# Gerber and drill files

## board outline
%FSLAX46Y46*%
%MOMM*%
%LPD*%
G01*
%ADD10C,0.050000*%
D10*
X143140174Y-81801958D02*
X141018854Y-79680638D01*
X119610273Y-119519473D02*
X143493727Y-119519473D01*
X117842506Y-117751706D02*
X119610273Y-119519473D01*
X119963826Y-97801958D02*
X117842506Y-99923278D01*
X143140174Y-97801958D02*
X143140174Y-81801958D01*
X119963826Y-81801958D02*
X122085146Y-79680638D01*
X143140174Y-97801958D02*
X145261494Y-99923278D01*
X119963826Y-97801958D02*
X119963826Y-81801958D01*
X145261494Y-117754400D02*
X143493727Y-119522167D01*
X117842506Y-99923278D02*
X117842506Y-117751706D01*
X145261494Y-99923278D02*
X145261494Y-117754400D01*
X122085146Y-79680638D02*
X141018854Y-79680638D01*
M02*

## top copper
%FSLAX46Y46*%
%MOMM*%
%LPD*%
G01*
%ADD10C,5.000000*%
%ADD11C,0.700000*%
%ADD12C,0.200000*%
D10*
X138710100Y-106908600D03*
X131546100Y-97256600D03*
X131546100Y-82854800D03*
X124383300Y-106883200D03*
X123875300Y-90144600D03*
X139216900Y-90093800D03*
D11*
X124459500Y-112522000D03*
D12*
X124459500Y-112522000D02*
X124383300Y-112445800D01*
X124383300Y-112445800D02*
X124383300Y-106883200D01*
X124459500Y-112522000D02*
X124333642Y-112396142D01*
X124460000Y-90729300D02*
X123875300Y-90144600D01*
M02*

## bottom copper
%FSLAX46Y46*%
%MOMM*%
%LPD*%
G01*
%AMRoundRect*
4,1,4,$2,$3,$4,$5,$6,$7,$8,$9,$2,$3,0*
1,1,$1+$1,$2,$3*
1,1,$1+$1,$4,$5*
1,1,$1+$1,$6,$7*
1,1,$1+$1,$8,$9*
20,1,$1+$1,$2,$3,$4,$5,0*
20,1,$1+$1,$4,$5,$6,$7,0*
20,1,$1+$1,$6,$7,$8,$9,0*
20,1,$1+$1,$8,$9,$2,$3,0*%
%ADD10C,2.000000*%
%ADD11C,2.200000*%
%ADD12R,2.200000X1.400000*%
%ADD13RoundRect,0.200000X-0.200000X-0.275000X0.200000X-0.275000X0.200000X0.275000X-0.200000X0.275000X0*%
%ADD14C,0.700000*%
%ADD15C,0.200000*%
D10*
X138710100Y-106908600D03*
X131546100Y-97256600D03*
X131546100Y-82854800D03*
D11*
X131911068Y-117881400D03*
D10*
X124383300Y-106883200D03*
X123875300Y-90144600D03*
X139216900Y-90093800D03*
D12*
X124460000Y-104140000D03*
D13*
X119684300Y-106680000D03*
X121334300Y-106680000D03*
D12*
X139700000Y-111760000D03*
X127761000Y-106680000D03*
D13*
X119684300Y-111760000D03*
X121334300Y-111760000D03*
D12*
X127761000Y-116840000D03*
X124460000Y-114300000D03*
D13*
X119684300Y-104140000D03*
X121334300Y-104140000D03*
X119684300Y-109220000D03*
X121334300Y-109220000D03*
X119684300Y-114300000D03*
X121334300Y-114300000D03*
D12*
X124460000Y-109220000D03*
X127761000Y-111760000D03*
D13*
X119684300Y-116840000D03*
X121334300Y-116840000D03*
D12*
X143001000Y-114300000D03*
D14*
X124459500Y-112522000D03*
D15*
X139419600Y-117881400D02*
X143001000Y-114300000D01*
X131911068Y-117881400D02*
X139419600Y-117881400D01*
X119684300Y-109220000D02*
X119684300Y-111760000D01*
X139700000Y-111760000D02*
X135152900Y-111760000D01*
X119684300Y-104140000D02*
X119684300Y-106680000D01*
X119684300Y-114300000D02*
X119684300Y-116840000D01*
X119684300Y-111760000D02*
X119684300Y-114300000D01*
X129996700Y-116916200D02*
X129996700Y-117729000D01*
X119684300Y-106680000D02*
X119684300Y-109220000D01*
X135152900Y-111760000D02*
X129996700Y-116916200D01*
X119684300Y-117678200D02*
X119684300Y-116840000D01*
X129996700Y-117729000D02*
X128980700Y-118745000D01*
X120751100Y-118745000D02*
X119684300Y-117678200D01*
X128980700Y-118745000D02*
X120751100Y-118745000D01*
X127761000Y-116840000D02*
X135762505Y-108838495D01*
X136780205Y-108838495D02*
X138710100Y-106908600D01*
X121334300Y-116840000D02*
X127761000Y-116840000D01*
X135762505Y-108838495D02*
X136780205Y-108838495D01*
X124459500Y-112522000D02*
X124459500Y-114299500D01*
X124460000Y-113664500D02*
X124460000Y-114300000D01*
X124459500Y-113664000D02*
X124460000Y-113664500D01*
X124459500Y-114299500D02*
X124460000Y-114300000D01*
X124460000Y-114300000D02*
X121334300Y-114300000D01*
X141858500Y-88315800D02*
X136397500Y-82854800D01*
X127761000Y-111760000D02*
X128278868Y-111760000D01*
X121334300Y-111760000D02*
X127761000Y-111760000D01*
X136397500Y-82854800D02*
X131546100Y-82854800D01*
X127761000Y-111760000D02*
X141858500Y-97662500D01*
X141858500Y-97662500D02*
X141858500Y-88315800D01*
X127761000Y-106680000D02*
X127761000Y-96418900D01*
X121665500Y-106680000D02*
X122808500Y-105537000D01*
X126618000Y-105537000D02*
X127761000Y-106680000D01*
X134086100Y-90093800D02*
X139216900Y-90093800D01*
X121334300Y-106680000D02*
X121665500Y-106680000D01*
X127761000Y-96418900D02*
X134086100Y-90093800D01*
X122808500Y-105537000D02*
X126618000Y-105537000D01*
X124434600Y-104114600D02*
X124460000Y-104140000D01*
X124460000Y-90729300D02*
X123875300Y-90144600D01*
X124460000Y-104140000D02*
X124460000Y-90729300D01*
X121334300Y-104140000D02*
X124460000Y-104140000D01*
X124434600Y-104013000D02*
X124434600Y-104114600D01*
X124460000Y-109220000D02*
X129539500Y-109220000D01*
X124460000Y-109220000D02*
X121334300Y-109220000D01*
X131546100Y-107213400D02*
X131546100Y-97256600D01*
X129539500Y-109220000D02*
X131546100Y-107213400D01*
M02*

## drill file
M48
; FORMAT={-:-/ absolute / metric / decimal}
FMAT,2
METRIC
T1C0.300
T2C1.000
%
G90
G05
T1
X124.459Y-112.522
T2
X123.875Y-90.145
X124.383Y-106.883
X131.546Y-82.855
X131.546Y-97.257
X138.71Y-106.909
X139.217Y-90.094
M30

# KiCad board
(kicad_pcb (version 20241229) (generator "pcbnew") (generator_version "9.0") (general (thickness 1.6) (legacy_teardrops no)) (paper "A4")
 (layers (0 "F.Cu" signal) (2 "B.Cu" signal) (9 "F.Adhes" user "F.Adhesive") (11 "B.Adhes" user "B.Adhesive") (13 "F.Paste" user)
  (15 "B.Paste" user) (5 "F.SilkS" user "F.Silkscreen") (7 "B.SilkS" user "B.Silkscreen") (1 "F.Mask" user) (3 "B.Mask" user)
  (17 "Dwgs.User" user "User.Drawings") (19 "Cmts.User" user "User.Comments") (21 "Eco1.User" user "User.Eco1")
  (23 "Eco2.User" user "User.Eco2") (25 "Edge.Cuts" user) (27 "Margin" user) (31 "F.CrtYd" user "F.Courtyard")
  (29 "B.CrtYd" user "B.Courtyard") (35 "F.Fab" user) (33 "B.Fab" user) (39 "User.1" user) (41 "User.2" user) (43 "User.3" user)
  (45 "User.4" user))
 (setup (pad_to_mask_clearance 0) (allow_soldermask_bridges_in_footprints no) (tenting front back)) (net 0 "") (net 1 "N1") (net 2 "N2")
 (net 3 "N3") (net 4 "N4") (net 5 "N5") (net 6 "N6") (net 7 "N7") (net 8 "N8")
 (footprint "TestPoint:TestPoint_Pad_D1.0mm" (layer "F.Cu") (at 138.7101 106.9086 90)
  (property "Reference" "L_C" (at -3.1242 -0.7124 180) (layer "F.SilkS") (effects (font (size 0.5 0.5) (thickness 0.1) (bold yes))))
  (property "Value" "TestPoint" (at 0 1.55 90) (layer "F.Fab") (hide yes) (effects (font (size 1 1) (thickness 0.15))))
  (pad "1" thru_hole circle (at 0 0 90) (size 5 5) (drill 1) (layers "*.Cu" "*.Mask") (remove_unused_layers no) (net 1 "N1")
   (padstack (mode front_inner_back) (layer "Inner" (shape circle) (size 5 5) (zone_connect -1))
    (layer "B.Cu" (shape circle) (size 2 2) (zone_connect -1)))))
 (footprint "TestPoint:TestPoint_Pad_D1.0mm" (layer "F.Cu") (at 131.5461 97.2566 90)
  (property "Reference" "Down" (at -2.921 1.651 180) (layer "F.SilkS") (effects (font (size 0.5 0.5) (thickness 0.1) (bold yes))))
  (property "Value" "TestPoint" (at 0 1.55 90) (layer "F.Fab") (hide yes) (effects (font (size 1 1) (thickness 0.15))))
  (pad "1" thru_hole circle (at 0 0 180) (size 5 5) (drill 1) (layers "*.Cu" "*.Mask") (remove_unused_layers no) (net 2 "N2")
   (padstack (mode front_inner_back) (layer "Inner" (shape circle) (size 5 5) (zone_connect -1))
    (layer "B.Cu" (shape circle) (size 2 2) (zone_connect -1)))))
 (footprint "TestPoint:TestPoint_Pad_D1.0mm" (layer "F.Cu") (at 131.5461 82.8548 90)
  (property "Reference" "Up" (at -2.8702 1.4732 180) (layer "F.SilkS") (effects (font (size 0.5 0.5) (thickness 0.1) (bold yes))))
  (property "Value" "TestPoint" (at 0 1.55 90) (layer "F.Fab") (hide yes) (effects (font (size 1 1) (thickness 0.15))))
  (pad "1" thru_hole circle (at 0 0) (size 5 5) (drill 1) (layers "*.Cu" "*.Mask") (remove_unused_layers no) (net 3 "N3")
   (padstack (mode front_inner_back) (layer "Inner" (shape circle) (size 5 5) (zone_connect -1))
    (layer "B.Cu" (shape circle) (size 2 2) (zone_connect -1)))))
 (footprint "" (layer "F.Cu") (at 131.911068 117.8814)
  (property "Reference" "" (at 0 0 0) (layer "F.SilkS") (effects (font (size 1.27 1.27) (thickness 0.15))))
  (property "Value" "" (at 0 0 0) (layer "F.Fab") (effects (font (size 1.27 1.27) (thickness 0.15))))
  (pad "1" smd circle (at 0 0 180) (size 2.2 2.2) (layers "B.Cu" "B.Mask") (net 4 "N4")))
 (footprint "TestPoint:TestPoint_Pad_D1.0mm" (layer "F.Cu") (at 124.3833 106.8832 90)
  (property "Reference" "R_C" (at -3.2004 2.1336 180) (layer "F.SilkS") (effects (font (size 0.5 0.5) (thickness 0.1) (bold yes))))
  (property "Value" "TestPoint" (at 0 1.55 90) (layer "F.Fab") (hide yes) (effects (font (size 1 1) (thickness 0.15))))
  (pad "1" thru_hole circle (at 0 0 90) (size 5 5) (drill 1) (layers "*.Cu" "*.Mask") (remove_unused_layers no) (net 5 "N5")
   (padstack (mode front_inner_back) (layer "Inner" (shape circle) (size 5 5) (zone_connect -1))
    (layer "B.Cu" (shape circle) (size 2 2) (zone_connect -1)))))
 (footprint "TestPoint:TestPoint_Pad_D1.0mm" (layer "F.Cu") (at 123.8753 90.1446 90)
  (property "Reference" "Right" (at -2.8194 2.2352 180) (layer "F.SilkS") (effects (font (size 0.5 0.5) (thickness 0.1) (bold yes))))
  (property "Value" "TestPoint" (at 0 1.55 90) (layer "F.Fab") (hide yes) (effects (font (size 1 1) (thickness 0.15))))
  (pad "1" thru_hole circle (at 0 0 270) (size 5 5) (drill 1) (layers "*.Cu" "*.Mask") (remove_unused_layers no) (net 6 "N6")
   (teardrops (best_length_ratio 0.5) (max_length 1) (best_width_ratio 0.7) (max_width 2) (curved_edges no) (filter_ratio 0.9) (enabled no)
    (allow_two_segments yes) (prefer_zone_connections yes))
   (padstack (mode front_inner_back) (layer "Inner" (shape circle) (size 5 5) (zone_connect -1))
    (layer "B.Cu" (shape circle) (size 2 2) (zone_connect -1)))))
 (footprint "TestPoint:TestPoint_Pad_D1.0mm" (layer "F.Cu") (at 139.2169 90.0938 90)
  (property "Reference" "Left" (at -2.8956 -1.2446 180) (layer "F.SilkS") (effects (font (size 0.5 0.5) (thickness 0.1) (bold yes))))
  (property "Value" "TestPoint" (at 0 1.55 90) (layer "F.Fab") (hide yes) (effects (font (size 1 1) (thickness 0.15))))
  (pad "1" thru_hole circle (at 0 0 90) (size 5 5) (drill 1) (layers "*.Cu" "*.Mask") (remove_unused_layers no) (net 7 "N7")
   (padstack (mode front_inner_back) (layer "Inner" (shape circle) (size 5 5) (zone_connect -1))
    (layer "B.Cu" (shape circle) (size 2 2) (zone_connect -1)))))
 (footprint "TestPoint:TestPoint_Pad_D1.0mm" (layer "B.Cu") (at 124.46 104.14 180)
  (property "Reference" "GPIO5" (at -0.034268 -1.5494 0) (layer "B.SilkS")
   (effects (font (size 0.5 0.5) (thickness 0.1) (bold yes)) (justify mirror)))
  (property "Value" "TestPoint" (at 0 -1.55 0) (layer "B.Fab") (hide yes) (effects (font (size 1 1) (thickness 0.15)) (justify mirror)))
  (pad "1" smd rect (at 0 0 180) (size 2.2 1.4) (layers "B.Cu" "B.Mask") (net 6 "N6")))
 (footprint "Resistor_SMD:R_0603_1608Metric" (layer "B.Cu") (at 120.5093 106.68)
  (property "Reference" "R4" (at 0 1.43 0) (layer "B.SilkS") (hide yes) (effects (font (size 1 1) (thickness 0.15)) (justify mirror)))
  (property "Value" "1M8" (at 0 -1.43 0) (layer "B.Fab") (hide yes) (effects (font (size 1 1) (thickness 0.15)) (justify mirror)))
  (pad "1" smd roundrect (at -0.825 0) (size 0.8 0.95) (layers "B.Cu" "B.Mask" "B.Paste") (roundrect_rratio 0.25) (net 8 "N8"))
  (pad "2" smd roundrect (at 0.825 0) (size 0.8 0.95) (layers "B.Cu" "B.Mask" "B.Paste") (roundrect_rratio 0.25) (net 7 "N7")))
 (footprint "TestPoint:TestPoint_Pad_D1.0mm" (layer "B.Cu") (at 139.7 111.76)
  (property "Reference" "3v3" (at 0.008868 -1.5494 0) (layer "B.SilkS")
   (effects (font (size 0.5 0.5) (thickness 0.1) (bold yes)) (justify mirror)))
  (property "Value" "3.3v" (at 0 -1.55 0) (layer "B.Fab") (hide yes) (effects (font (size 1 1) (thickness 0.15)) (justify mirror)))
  (pad "1" smd rect (at 0 0) (size 2.2 1.4) (layers "B.Cu" "B.Mask") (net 8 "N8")))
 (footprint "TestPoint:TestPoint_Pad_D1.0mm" (layer "B.Cu") (at 127.761 106.68 180)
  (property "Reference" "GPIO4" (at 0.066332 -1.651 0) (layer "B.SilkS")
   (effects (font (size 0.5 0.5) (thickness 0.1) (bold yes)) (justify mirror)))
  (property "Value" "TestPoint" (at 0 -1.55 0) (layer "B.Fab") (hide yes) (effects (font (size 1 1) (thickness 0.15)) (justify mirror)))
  (pad "1" smd rect (at 0 0 180) (size 2.2 1.4) (layers "B.Cu" "B.Mask") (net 7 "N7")))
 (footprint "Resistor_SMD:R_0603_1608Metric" (layer "B.Cu") (at 120.5093 111.76)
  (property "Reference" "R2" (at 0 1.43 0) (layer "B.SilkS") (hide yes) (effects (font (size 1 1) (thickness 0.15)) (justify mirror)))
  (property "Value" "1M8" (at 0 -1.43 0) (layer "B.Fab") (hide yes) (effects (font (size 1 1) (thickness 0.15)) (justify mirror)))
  (pad "1" smd roundrect (at -0.825 0) (size 0.8 0.95) (layers "B.Cu" "B.Mask" "B.Paste") (roundrect_rratio 0.25) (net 8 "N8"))
  (pad "2" smd roundrect (at 0.825 0) (size 0.8 0.95) (layers "B.Cu" "B.Mask" "B.Paste") (roundrect_rratio 0.25) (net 3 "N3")))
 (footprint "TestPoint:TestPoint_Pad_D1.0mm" (layer "B.Cu") (at 127.761 116.84 180)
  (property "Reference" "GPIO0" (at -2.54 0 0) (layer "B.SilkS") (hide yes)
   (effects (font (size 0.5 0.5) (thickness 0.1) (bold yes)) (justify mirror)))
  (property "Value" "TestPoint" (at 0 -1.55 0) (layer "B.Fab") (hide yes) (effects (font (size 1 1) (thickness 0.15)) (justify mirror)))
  (pad "1" smd rect (at 0 0 180) (size 2.2 1.4) (layers "B.Cu" "B.Mask") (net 1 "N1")))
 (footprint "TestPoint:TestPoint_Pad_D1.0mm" (layer "B.Cu") (at 124.46 114.3 180)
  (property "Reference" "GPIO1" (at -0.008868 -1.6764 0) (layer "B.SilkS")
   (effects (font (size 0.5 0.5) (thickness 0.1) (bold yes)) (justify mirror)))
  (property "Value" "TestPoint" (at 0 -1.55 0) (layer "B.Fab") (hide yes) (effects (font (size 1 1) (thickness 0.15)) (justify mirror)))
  (pad "1" smd rect (at 0 0 180) (size 2.2 1.4) (layers "B.Cu" "B.Mask") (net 5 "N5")))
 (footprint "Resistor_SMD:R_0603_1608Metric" (layer "B.Cu") (at 120.5093 104.14)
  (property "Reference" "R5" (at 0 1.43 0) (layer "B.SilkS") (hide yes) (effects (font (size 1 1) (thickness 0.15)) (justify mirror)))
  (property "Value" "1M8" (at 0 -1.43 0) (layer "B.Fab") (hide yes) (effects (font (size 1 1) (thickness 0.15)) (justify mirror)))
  (pad "1" smd roundrect (at -0.825 0) (size 0.8 0.95) (layers "B.Cu" "B.Mask" "B.Paste") (roundrect_rratio 0.25) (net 8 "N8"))
  (pad "2" smd roundrect (at 0.825 0) (size 0.8 0.95) (layers "B.Cu" "B.Mask" "B.Paste") (roundrect_rratio 0.25) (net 6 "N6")))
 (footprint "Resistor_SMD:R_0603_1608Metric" (layer "B.Cu") (at 120.5093 109.22)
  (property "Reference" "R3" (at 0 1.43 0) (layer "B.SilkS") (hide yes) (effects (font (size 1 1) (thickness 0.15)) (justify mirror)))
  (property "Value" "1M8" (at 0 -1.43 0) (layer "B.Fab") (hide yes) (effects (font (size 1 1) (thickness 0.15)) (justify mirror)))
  (pad "1" smd roundrect (at -0.825 0) (size 0.8 0.95) (layers "B.Cu" "B.Mask" "B.Paste") (roundrect_rratio 0.25) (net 8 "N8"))
  (pad "2" smd roundrect (at 0.825 0) (size 0.8 0.95) (layers "B.Cu" "B.Mask" "B.Paste") (roundrect_rratio 0.25) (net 2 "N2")))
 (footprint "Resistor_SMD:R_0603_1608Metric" (layer "B.Cu") (at 120.5093 114.3)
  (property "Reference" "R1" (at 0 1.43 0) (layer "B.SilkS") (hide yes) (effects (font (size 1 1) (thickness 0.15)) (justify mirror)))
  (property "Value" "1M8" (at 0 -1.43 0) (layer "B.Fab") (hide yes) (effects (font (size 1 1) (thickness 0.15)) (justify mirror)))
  (pad "1" smd roundrect (at -0.825 0) (size 0.8 0.95) (layers "B.Cu" "B.Mask" "B.Paste") (roundrect_rratio 0.25) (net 8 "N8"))
  (pad "2" smd roundrect (at 0.825 0) (size 0.8 0.95) (layers "B.Cu" "B.Mask" "B.Paste") (roundrect_rratio 0.25) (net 5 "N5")))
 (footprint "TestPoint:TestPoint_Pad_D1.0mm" (layer "B.Cu") (at 124.46 109.22 180)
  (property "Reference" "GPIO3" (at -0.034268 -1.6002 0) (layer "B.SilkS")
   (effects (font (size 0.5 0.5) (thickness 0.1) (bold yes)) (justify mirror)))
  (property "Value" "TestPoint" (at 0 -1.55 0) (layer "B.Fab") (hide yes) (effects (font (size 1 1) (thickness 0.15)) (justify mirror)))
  (pad "1" smd rect (at 0 0 180) (size 2.2 1.4) (layers "B.Cu" "B.Mask") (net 2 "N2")))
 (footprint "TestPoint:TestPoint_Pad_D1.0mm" (layer "B.Cu") (at 127.761 111.76 180)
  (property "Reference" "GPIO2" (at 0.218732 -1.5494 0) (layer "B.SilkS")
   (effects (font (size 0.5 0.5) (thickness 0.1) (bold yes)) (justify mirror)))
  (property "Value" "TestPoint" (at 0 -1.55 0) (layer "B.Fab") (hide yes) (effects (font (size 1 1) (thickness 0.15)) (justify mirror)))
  (pad "1" smd rect (at 0 0 180) (size 2.2 1.4) (layers "B.Cu" "B.Mask") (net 3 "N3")))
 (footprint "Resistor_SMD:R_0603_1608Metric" (layer "B.Cu") (at 120.5093 116.84)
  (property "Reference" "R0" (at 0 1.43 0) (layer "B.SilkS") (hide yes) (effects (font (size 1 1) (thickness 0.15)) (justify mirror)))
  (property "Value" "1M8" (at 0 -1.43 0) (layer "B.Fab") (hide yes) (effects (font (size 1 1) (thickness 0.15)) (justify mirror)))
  (pad "1" smd roundrect (at -0.825 0) (size 0.8 0.95) (layers "B.Cu" "B.Mask" "B.Paste") (roundrect_rratio 0.25) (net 8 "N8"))
  (pad "2" smd roundrect (at 0.825 0) (size 0.8 0.95) (layers "B.Cu" "B.Mask" "B.Paste") (roundrect_rratio 0.25) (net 1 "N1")))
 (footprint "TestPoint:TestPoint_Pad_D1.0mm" (layer "B.Cu") (at 143.001 114.3)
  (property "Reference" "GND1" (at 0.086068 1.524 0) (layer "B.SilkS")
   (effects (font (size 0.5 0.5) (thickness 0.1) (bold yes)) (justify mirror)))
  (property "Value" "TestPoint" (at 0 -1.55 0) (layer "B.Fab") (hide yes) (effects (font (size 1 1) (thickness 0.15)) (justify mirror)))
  (pad "1" smd rect (at 0 0) (size 2.2 1.4) (layers "B.Cu" "B.Mask") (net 4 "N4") (clearance 0.1)))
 (gr_line (start 143.140174 81.801958) (end 141.018854 79.680638) (stroke (width 0.05) (type solid)) (layer "Edge.Cuts"))
 (gr_line (start 119.610273 119.519473) (end 143.493727 119.519473) (stroke (width 0.05) (type default)) (layer "Edge.Cuts"))
 (gr_line (start 117.842506 117.751706) (end 119.610273 119.519473) (stroke (width 0.05) (type solid)) (layer "Edge.Cuts"))
 (gr_line (start 119.963826 97.801958) (end 117.842506 99.923278) (stroke (width 0.05) (type solid)) (layer "Edge.Cuts"))
 (gr_line (start 143.140174 97.801958) (end 143.140174 81.801958) (stroke (width 0.05) (type solid)) (layer "Edge.Cuts"))
 (gr_line (start 119.963826 81.801958) (end 122.085146 79.680638) (stroke (width 0.05) (type solid)) (layer "Edge.Cuts"))
 (gr_line (start 143.140174 97.801958) (end 145.261494 99.923278) (stroke (width 0.05) (type solid)) (layer "Edge.Cuts"))
 (gr_line (start 119.963826 97.801958) (end 119.963826 81.801958) (stroke (width 0.05) (type solid)) (layer "Edge.Cuts"))
 (gr_line (start 145.261494 117.7544) (end 143.493727 119.522167) (stroke (width 0.05) (type solid)) (layer "Edge.Cuts"))
 (gr_line (start 117.842506 99.923278) (end 117.842506 117.751706) (stroke (width 0.05) (type default)) (layer "Edge.Cuts"))
 (gr_line (start 145.261494 99.923278) (end 145.261494 117.7544) (stroke (width 0.05) (type default)) (layer "Edge.Cuts"))
 (gr_line (start 122.085146 79.680638) (end 141.018854 79.680638) (stroke (width 0.05) (type default)) (layer "Edge.Cuts"))
 (segment (start 139.4196 117.8814) (end 143.001 114.3) (width 0.2) (layer "B.Cu") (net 4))
 (segment (start 131.911068 117.8814) (end 139.4196 117.8814) (width 0.2) (layer "B.Cu") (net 4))
 (segment (start 119.6843 109.22) (end 119.6843 111.76) (width 0.2) (layer "B.Cu") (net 8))
 (segment (start 139.7 111.76) (end 135.1529 111.76) (width 0.2) (layer "B.Cu") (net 8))
 (segment (start 119.6843 104.14) (end 119.6843 106.68) (width 0.2) (layer "B.Cu") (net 8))
 (segment (start 119.6843 114.3) (end 119.6843 116.84) (width 0.2) (layer "B.Cu") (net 8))
 (segment (start 119.6843 111.76) (end 119.6843 114.3) (width 0.2) (layer "B.Cu") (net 8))
 (segment (start 129.9967 116.9162) (end 129.9967 117.729) (width 0.2) (layer "B.Cu") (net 8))
 (segment (start 119.6843 106.68) (end 119.6843 109.22) (width 0.2) (layer "B.Cu") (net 8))
 (segment (start 135.1529 111.76) (end 129.9967 116.9162) (width 0.2) (layer "B.Cu") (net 8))
 (segment (start 119.6843 117.6782) (end 119.6843 116.84) (width 0.2) (layer "B.Cu") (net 8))
 (segment (start 129.9967 117.729) (end 128.9807 118.745) (width 0.2) (layer "B.Cu") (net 8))
 (segment (start 120.7511 118.745) (end 119.6843 117.6782) (width 0.2) (layer "B.Cu") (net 8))
 (segment (start 128.9807 118.745) (end 120.7511 118.745) (width 0.2) (layer "B.Cu") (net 8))
 (segment (start 127.761 116.84) (end 135.762505 108.838495) (width 0.2) (layer "B.Cu") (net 1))
 (segment (start 136.780205 108.838495) (end 138.7101 106.9086) (width 0.2) (layer "B.Cu") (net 1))
 (segment (start 121.3343 116.84) (end 127.761 116.84) (width 0.2) (layer "B.Cu") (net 1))
 (segment (start 135.762505 108.838495) (end 136.780205 108.838495) (width 0.2) (layer "B.Cu") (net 1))
 (segment (start 124.4595 112.522) (end 124.3833 112.4458) (width 0.2) (layer "F.Cu") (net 5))
 (segment (start 124.3833 112.4458) (end 124.3833 106.8832) (width 0.2) (layer "F.Cu") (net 5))
 (segment (start 124.4595 112.522) (end 124.333642 112.396142) (width 0.2) (layer "F.Cu") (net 5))
 (via (at 124.4595 112.522) (size 0.7) (drill 0.3) (layers "F.Cu" "B.Cu") (tenting front back) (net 5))
 (segment (start 124.4595 112.522) (end 124.4595 114.2995) (width 0.2) (layer "B.Cu") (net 5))
 (segment (start 124.46 113.6645) (end 124.46 114.3) (width 0.2) (layer "B.Cu") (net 5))
 (segment (start 124.4595 113.664) (end 124.46 113.6645) (width 0.2) (layer "B.Cu") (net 5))
 (segment (start 124.4595 114.2995) (end 124.46 114.3) (width 0.2) (layer "B.Cu") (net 5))
 (segment (start 124.46 114.3) (end 121.3343 114.3) (width 0.2) (layer "B.Cu") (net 5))
 (segment (start 141.8585 88.3158) (end 136.3975 82.8548) (width 0.2) (layer "B.Cu") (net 3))
 (segment (start 127.761 111.76) (end 128.278868 111.76) (width 0.2) (layer "B.Cu") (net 3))
 (segment (start 121.3343 111.76) (end 127.761 111.76) (width 0.2) (layer "B.Cu") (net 3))
 (segment (start 136.3975 82.8548) (end 131.5461 82.8548) (width 0.2) (layer "B.Cu") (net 3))
 (segment (start 127.761 111.76) (end 141.8585 97.6625) (width 0.2) (layer "B.Cu") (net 3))
 (segment (start 141.8585 97.6625) (end 141.8585 88.3158) (width 0.2) (layer "B.Cu") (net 3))
 (segment (start 127.761 106.68) (end 127.761 96.4189) (width 0.2) (layer "B.Cu") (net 7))
 (segment (start 121.6655 106.68) (end 122.8085 105.537) (width 0.2) (layer "B.Cu") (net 7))
 (segment (start 126.618 105.537) (end 127.761 106.68) (width 0.2) (layer "B.Cu") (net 7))
 (segment (start 134.0861 90.0938) (end 139.2169 90.0938) (width 0.2) (layer "B.Cu") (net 7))
 (segment (start 121.3343 106.68) (end 121.6655 106.68) (width 0.2) (layer "B.Cu") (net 7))
 (segment (start 127.761 96.4189) (end 134.0861 90.0938) (width 0.2) (layer "B.Cu") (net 7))
 (segment (start 122.8085 105.537) (end 126.618 105.537) (width 0.2) (layer "B.Cu") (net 7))
 (segment (start 124.46 90.7293) (end 123.8753 90.1446) (width 0.2) (layer "F.Cu") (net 6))
 (segment (start 124.4346 104.1146) (end 124.46 104.14) (width 0.2) (layer "B.Cu") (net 6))
 (segment (start 124.46 90.7293) (end 123.8753 90.1446) (width 0.2) (layer "B.Cu") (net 6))
 (segment (start 124.46 104.14) (end 124.46 90.7293) (width 0.2) (layer "B.Cu") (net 6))
 (segment (start 121.3343 104.14) (end 124.46 104.14) (width 0.2) (layer "B.Cu") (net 6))
 (segment (start 124.4346 104.013) (end 124.4346 104.1146) (width 0.2) (layer "B.Cu") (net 6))
 (segment (start 124.46 109.22) (end 129.5395 109.22) (width 0.2) (layer "B.Cu") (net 2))
 (segment (start 124.46 109.22) (end 121.3343 109.22) (width 0.2) (layer "B.Cu") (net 2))
 (segment (start 131.5461 107.2134) (end 131.5461 97.2566) (width 0.2) (layer "B.Cu") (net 2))
 (segment (start 129.5395 109.22) (end 131.5461 107.2134) (width 0.2) (layer "B.Cu") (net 2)))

